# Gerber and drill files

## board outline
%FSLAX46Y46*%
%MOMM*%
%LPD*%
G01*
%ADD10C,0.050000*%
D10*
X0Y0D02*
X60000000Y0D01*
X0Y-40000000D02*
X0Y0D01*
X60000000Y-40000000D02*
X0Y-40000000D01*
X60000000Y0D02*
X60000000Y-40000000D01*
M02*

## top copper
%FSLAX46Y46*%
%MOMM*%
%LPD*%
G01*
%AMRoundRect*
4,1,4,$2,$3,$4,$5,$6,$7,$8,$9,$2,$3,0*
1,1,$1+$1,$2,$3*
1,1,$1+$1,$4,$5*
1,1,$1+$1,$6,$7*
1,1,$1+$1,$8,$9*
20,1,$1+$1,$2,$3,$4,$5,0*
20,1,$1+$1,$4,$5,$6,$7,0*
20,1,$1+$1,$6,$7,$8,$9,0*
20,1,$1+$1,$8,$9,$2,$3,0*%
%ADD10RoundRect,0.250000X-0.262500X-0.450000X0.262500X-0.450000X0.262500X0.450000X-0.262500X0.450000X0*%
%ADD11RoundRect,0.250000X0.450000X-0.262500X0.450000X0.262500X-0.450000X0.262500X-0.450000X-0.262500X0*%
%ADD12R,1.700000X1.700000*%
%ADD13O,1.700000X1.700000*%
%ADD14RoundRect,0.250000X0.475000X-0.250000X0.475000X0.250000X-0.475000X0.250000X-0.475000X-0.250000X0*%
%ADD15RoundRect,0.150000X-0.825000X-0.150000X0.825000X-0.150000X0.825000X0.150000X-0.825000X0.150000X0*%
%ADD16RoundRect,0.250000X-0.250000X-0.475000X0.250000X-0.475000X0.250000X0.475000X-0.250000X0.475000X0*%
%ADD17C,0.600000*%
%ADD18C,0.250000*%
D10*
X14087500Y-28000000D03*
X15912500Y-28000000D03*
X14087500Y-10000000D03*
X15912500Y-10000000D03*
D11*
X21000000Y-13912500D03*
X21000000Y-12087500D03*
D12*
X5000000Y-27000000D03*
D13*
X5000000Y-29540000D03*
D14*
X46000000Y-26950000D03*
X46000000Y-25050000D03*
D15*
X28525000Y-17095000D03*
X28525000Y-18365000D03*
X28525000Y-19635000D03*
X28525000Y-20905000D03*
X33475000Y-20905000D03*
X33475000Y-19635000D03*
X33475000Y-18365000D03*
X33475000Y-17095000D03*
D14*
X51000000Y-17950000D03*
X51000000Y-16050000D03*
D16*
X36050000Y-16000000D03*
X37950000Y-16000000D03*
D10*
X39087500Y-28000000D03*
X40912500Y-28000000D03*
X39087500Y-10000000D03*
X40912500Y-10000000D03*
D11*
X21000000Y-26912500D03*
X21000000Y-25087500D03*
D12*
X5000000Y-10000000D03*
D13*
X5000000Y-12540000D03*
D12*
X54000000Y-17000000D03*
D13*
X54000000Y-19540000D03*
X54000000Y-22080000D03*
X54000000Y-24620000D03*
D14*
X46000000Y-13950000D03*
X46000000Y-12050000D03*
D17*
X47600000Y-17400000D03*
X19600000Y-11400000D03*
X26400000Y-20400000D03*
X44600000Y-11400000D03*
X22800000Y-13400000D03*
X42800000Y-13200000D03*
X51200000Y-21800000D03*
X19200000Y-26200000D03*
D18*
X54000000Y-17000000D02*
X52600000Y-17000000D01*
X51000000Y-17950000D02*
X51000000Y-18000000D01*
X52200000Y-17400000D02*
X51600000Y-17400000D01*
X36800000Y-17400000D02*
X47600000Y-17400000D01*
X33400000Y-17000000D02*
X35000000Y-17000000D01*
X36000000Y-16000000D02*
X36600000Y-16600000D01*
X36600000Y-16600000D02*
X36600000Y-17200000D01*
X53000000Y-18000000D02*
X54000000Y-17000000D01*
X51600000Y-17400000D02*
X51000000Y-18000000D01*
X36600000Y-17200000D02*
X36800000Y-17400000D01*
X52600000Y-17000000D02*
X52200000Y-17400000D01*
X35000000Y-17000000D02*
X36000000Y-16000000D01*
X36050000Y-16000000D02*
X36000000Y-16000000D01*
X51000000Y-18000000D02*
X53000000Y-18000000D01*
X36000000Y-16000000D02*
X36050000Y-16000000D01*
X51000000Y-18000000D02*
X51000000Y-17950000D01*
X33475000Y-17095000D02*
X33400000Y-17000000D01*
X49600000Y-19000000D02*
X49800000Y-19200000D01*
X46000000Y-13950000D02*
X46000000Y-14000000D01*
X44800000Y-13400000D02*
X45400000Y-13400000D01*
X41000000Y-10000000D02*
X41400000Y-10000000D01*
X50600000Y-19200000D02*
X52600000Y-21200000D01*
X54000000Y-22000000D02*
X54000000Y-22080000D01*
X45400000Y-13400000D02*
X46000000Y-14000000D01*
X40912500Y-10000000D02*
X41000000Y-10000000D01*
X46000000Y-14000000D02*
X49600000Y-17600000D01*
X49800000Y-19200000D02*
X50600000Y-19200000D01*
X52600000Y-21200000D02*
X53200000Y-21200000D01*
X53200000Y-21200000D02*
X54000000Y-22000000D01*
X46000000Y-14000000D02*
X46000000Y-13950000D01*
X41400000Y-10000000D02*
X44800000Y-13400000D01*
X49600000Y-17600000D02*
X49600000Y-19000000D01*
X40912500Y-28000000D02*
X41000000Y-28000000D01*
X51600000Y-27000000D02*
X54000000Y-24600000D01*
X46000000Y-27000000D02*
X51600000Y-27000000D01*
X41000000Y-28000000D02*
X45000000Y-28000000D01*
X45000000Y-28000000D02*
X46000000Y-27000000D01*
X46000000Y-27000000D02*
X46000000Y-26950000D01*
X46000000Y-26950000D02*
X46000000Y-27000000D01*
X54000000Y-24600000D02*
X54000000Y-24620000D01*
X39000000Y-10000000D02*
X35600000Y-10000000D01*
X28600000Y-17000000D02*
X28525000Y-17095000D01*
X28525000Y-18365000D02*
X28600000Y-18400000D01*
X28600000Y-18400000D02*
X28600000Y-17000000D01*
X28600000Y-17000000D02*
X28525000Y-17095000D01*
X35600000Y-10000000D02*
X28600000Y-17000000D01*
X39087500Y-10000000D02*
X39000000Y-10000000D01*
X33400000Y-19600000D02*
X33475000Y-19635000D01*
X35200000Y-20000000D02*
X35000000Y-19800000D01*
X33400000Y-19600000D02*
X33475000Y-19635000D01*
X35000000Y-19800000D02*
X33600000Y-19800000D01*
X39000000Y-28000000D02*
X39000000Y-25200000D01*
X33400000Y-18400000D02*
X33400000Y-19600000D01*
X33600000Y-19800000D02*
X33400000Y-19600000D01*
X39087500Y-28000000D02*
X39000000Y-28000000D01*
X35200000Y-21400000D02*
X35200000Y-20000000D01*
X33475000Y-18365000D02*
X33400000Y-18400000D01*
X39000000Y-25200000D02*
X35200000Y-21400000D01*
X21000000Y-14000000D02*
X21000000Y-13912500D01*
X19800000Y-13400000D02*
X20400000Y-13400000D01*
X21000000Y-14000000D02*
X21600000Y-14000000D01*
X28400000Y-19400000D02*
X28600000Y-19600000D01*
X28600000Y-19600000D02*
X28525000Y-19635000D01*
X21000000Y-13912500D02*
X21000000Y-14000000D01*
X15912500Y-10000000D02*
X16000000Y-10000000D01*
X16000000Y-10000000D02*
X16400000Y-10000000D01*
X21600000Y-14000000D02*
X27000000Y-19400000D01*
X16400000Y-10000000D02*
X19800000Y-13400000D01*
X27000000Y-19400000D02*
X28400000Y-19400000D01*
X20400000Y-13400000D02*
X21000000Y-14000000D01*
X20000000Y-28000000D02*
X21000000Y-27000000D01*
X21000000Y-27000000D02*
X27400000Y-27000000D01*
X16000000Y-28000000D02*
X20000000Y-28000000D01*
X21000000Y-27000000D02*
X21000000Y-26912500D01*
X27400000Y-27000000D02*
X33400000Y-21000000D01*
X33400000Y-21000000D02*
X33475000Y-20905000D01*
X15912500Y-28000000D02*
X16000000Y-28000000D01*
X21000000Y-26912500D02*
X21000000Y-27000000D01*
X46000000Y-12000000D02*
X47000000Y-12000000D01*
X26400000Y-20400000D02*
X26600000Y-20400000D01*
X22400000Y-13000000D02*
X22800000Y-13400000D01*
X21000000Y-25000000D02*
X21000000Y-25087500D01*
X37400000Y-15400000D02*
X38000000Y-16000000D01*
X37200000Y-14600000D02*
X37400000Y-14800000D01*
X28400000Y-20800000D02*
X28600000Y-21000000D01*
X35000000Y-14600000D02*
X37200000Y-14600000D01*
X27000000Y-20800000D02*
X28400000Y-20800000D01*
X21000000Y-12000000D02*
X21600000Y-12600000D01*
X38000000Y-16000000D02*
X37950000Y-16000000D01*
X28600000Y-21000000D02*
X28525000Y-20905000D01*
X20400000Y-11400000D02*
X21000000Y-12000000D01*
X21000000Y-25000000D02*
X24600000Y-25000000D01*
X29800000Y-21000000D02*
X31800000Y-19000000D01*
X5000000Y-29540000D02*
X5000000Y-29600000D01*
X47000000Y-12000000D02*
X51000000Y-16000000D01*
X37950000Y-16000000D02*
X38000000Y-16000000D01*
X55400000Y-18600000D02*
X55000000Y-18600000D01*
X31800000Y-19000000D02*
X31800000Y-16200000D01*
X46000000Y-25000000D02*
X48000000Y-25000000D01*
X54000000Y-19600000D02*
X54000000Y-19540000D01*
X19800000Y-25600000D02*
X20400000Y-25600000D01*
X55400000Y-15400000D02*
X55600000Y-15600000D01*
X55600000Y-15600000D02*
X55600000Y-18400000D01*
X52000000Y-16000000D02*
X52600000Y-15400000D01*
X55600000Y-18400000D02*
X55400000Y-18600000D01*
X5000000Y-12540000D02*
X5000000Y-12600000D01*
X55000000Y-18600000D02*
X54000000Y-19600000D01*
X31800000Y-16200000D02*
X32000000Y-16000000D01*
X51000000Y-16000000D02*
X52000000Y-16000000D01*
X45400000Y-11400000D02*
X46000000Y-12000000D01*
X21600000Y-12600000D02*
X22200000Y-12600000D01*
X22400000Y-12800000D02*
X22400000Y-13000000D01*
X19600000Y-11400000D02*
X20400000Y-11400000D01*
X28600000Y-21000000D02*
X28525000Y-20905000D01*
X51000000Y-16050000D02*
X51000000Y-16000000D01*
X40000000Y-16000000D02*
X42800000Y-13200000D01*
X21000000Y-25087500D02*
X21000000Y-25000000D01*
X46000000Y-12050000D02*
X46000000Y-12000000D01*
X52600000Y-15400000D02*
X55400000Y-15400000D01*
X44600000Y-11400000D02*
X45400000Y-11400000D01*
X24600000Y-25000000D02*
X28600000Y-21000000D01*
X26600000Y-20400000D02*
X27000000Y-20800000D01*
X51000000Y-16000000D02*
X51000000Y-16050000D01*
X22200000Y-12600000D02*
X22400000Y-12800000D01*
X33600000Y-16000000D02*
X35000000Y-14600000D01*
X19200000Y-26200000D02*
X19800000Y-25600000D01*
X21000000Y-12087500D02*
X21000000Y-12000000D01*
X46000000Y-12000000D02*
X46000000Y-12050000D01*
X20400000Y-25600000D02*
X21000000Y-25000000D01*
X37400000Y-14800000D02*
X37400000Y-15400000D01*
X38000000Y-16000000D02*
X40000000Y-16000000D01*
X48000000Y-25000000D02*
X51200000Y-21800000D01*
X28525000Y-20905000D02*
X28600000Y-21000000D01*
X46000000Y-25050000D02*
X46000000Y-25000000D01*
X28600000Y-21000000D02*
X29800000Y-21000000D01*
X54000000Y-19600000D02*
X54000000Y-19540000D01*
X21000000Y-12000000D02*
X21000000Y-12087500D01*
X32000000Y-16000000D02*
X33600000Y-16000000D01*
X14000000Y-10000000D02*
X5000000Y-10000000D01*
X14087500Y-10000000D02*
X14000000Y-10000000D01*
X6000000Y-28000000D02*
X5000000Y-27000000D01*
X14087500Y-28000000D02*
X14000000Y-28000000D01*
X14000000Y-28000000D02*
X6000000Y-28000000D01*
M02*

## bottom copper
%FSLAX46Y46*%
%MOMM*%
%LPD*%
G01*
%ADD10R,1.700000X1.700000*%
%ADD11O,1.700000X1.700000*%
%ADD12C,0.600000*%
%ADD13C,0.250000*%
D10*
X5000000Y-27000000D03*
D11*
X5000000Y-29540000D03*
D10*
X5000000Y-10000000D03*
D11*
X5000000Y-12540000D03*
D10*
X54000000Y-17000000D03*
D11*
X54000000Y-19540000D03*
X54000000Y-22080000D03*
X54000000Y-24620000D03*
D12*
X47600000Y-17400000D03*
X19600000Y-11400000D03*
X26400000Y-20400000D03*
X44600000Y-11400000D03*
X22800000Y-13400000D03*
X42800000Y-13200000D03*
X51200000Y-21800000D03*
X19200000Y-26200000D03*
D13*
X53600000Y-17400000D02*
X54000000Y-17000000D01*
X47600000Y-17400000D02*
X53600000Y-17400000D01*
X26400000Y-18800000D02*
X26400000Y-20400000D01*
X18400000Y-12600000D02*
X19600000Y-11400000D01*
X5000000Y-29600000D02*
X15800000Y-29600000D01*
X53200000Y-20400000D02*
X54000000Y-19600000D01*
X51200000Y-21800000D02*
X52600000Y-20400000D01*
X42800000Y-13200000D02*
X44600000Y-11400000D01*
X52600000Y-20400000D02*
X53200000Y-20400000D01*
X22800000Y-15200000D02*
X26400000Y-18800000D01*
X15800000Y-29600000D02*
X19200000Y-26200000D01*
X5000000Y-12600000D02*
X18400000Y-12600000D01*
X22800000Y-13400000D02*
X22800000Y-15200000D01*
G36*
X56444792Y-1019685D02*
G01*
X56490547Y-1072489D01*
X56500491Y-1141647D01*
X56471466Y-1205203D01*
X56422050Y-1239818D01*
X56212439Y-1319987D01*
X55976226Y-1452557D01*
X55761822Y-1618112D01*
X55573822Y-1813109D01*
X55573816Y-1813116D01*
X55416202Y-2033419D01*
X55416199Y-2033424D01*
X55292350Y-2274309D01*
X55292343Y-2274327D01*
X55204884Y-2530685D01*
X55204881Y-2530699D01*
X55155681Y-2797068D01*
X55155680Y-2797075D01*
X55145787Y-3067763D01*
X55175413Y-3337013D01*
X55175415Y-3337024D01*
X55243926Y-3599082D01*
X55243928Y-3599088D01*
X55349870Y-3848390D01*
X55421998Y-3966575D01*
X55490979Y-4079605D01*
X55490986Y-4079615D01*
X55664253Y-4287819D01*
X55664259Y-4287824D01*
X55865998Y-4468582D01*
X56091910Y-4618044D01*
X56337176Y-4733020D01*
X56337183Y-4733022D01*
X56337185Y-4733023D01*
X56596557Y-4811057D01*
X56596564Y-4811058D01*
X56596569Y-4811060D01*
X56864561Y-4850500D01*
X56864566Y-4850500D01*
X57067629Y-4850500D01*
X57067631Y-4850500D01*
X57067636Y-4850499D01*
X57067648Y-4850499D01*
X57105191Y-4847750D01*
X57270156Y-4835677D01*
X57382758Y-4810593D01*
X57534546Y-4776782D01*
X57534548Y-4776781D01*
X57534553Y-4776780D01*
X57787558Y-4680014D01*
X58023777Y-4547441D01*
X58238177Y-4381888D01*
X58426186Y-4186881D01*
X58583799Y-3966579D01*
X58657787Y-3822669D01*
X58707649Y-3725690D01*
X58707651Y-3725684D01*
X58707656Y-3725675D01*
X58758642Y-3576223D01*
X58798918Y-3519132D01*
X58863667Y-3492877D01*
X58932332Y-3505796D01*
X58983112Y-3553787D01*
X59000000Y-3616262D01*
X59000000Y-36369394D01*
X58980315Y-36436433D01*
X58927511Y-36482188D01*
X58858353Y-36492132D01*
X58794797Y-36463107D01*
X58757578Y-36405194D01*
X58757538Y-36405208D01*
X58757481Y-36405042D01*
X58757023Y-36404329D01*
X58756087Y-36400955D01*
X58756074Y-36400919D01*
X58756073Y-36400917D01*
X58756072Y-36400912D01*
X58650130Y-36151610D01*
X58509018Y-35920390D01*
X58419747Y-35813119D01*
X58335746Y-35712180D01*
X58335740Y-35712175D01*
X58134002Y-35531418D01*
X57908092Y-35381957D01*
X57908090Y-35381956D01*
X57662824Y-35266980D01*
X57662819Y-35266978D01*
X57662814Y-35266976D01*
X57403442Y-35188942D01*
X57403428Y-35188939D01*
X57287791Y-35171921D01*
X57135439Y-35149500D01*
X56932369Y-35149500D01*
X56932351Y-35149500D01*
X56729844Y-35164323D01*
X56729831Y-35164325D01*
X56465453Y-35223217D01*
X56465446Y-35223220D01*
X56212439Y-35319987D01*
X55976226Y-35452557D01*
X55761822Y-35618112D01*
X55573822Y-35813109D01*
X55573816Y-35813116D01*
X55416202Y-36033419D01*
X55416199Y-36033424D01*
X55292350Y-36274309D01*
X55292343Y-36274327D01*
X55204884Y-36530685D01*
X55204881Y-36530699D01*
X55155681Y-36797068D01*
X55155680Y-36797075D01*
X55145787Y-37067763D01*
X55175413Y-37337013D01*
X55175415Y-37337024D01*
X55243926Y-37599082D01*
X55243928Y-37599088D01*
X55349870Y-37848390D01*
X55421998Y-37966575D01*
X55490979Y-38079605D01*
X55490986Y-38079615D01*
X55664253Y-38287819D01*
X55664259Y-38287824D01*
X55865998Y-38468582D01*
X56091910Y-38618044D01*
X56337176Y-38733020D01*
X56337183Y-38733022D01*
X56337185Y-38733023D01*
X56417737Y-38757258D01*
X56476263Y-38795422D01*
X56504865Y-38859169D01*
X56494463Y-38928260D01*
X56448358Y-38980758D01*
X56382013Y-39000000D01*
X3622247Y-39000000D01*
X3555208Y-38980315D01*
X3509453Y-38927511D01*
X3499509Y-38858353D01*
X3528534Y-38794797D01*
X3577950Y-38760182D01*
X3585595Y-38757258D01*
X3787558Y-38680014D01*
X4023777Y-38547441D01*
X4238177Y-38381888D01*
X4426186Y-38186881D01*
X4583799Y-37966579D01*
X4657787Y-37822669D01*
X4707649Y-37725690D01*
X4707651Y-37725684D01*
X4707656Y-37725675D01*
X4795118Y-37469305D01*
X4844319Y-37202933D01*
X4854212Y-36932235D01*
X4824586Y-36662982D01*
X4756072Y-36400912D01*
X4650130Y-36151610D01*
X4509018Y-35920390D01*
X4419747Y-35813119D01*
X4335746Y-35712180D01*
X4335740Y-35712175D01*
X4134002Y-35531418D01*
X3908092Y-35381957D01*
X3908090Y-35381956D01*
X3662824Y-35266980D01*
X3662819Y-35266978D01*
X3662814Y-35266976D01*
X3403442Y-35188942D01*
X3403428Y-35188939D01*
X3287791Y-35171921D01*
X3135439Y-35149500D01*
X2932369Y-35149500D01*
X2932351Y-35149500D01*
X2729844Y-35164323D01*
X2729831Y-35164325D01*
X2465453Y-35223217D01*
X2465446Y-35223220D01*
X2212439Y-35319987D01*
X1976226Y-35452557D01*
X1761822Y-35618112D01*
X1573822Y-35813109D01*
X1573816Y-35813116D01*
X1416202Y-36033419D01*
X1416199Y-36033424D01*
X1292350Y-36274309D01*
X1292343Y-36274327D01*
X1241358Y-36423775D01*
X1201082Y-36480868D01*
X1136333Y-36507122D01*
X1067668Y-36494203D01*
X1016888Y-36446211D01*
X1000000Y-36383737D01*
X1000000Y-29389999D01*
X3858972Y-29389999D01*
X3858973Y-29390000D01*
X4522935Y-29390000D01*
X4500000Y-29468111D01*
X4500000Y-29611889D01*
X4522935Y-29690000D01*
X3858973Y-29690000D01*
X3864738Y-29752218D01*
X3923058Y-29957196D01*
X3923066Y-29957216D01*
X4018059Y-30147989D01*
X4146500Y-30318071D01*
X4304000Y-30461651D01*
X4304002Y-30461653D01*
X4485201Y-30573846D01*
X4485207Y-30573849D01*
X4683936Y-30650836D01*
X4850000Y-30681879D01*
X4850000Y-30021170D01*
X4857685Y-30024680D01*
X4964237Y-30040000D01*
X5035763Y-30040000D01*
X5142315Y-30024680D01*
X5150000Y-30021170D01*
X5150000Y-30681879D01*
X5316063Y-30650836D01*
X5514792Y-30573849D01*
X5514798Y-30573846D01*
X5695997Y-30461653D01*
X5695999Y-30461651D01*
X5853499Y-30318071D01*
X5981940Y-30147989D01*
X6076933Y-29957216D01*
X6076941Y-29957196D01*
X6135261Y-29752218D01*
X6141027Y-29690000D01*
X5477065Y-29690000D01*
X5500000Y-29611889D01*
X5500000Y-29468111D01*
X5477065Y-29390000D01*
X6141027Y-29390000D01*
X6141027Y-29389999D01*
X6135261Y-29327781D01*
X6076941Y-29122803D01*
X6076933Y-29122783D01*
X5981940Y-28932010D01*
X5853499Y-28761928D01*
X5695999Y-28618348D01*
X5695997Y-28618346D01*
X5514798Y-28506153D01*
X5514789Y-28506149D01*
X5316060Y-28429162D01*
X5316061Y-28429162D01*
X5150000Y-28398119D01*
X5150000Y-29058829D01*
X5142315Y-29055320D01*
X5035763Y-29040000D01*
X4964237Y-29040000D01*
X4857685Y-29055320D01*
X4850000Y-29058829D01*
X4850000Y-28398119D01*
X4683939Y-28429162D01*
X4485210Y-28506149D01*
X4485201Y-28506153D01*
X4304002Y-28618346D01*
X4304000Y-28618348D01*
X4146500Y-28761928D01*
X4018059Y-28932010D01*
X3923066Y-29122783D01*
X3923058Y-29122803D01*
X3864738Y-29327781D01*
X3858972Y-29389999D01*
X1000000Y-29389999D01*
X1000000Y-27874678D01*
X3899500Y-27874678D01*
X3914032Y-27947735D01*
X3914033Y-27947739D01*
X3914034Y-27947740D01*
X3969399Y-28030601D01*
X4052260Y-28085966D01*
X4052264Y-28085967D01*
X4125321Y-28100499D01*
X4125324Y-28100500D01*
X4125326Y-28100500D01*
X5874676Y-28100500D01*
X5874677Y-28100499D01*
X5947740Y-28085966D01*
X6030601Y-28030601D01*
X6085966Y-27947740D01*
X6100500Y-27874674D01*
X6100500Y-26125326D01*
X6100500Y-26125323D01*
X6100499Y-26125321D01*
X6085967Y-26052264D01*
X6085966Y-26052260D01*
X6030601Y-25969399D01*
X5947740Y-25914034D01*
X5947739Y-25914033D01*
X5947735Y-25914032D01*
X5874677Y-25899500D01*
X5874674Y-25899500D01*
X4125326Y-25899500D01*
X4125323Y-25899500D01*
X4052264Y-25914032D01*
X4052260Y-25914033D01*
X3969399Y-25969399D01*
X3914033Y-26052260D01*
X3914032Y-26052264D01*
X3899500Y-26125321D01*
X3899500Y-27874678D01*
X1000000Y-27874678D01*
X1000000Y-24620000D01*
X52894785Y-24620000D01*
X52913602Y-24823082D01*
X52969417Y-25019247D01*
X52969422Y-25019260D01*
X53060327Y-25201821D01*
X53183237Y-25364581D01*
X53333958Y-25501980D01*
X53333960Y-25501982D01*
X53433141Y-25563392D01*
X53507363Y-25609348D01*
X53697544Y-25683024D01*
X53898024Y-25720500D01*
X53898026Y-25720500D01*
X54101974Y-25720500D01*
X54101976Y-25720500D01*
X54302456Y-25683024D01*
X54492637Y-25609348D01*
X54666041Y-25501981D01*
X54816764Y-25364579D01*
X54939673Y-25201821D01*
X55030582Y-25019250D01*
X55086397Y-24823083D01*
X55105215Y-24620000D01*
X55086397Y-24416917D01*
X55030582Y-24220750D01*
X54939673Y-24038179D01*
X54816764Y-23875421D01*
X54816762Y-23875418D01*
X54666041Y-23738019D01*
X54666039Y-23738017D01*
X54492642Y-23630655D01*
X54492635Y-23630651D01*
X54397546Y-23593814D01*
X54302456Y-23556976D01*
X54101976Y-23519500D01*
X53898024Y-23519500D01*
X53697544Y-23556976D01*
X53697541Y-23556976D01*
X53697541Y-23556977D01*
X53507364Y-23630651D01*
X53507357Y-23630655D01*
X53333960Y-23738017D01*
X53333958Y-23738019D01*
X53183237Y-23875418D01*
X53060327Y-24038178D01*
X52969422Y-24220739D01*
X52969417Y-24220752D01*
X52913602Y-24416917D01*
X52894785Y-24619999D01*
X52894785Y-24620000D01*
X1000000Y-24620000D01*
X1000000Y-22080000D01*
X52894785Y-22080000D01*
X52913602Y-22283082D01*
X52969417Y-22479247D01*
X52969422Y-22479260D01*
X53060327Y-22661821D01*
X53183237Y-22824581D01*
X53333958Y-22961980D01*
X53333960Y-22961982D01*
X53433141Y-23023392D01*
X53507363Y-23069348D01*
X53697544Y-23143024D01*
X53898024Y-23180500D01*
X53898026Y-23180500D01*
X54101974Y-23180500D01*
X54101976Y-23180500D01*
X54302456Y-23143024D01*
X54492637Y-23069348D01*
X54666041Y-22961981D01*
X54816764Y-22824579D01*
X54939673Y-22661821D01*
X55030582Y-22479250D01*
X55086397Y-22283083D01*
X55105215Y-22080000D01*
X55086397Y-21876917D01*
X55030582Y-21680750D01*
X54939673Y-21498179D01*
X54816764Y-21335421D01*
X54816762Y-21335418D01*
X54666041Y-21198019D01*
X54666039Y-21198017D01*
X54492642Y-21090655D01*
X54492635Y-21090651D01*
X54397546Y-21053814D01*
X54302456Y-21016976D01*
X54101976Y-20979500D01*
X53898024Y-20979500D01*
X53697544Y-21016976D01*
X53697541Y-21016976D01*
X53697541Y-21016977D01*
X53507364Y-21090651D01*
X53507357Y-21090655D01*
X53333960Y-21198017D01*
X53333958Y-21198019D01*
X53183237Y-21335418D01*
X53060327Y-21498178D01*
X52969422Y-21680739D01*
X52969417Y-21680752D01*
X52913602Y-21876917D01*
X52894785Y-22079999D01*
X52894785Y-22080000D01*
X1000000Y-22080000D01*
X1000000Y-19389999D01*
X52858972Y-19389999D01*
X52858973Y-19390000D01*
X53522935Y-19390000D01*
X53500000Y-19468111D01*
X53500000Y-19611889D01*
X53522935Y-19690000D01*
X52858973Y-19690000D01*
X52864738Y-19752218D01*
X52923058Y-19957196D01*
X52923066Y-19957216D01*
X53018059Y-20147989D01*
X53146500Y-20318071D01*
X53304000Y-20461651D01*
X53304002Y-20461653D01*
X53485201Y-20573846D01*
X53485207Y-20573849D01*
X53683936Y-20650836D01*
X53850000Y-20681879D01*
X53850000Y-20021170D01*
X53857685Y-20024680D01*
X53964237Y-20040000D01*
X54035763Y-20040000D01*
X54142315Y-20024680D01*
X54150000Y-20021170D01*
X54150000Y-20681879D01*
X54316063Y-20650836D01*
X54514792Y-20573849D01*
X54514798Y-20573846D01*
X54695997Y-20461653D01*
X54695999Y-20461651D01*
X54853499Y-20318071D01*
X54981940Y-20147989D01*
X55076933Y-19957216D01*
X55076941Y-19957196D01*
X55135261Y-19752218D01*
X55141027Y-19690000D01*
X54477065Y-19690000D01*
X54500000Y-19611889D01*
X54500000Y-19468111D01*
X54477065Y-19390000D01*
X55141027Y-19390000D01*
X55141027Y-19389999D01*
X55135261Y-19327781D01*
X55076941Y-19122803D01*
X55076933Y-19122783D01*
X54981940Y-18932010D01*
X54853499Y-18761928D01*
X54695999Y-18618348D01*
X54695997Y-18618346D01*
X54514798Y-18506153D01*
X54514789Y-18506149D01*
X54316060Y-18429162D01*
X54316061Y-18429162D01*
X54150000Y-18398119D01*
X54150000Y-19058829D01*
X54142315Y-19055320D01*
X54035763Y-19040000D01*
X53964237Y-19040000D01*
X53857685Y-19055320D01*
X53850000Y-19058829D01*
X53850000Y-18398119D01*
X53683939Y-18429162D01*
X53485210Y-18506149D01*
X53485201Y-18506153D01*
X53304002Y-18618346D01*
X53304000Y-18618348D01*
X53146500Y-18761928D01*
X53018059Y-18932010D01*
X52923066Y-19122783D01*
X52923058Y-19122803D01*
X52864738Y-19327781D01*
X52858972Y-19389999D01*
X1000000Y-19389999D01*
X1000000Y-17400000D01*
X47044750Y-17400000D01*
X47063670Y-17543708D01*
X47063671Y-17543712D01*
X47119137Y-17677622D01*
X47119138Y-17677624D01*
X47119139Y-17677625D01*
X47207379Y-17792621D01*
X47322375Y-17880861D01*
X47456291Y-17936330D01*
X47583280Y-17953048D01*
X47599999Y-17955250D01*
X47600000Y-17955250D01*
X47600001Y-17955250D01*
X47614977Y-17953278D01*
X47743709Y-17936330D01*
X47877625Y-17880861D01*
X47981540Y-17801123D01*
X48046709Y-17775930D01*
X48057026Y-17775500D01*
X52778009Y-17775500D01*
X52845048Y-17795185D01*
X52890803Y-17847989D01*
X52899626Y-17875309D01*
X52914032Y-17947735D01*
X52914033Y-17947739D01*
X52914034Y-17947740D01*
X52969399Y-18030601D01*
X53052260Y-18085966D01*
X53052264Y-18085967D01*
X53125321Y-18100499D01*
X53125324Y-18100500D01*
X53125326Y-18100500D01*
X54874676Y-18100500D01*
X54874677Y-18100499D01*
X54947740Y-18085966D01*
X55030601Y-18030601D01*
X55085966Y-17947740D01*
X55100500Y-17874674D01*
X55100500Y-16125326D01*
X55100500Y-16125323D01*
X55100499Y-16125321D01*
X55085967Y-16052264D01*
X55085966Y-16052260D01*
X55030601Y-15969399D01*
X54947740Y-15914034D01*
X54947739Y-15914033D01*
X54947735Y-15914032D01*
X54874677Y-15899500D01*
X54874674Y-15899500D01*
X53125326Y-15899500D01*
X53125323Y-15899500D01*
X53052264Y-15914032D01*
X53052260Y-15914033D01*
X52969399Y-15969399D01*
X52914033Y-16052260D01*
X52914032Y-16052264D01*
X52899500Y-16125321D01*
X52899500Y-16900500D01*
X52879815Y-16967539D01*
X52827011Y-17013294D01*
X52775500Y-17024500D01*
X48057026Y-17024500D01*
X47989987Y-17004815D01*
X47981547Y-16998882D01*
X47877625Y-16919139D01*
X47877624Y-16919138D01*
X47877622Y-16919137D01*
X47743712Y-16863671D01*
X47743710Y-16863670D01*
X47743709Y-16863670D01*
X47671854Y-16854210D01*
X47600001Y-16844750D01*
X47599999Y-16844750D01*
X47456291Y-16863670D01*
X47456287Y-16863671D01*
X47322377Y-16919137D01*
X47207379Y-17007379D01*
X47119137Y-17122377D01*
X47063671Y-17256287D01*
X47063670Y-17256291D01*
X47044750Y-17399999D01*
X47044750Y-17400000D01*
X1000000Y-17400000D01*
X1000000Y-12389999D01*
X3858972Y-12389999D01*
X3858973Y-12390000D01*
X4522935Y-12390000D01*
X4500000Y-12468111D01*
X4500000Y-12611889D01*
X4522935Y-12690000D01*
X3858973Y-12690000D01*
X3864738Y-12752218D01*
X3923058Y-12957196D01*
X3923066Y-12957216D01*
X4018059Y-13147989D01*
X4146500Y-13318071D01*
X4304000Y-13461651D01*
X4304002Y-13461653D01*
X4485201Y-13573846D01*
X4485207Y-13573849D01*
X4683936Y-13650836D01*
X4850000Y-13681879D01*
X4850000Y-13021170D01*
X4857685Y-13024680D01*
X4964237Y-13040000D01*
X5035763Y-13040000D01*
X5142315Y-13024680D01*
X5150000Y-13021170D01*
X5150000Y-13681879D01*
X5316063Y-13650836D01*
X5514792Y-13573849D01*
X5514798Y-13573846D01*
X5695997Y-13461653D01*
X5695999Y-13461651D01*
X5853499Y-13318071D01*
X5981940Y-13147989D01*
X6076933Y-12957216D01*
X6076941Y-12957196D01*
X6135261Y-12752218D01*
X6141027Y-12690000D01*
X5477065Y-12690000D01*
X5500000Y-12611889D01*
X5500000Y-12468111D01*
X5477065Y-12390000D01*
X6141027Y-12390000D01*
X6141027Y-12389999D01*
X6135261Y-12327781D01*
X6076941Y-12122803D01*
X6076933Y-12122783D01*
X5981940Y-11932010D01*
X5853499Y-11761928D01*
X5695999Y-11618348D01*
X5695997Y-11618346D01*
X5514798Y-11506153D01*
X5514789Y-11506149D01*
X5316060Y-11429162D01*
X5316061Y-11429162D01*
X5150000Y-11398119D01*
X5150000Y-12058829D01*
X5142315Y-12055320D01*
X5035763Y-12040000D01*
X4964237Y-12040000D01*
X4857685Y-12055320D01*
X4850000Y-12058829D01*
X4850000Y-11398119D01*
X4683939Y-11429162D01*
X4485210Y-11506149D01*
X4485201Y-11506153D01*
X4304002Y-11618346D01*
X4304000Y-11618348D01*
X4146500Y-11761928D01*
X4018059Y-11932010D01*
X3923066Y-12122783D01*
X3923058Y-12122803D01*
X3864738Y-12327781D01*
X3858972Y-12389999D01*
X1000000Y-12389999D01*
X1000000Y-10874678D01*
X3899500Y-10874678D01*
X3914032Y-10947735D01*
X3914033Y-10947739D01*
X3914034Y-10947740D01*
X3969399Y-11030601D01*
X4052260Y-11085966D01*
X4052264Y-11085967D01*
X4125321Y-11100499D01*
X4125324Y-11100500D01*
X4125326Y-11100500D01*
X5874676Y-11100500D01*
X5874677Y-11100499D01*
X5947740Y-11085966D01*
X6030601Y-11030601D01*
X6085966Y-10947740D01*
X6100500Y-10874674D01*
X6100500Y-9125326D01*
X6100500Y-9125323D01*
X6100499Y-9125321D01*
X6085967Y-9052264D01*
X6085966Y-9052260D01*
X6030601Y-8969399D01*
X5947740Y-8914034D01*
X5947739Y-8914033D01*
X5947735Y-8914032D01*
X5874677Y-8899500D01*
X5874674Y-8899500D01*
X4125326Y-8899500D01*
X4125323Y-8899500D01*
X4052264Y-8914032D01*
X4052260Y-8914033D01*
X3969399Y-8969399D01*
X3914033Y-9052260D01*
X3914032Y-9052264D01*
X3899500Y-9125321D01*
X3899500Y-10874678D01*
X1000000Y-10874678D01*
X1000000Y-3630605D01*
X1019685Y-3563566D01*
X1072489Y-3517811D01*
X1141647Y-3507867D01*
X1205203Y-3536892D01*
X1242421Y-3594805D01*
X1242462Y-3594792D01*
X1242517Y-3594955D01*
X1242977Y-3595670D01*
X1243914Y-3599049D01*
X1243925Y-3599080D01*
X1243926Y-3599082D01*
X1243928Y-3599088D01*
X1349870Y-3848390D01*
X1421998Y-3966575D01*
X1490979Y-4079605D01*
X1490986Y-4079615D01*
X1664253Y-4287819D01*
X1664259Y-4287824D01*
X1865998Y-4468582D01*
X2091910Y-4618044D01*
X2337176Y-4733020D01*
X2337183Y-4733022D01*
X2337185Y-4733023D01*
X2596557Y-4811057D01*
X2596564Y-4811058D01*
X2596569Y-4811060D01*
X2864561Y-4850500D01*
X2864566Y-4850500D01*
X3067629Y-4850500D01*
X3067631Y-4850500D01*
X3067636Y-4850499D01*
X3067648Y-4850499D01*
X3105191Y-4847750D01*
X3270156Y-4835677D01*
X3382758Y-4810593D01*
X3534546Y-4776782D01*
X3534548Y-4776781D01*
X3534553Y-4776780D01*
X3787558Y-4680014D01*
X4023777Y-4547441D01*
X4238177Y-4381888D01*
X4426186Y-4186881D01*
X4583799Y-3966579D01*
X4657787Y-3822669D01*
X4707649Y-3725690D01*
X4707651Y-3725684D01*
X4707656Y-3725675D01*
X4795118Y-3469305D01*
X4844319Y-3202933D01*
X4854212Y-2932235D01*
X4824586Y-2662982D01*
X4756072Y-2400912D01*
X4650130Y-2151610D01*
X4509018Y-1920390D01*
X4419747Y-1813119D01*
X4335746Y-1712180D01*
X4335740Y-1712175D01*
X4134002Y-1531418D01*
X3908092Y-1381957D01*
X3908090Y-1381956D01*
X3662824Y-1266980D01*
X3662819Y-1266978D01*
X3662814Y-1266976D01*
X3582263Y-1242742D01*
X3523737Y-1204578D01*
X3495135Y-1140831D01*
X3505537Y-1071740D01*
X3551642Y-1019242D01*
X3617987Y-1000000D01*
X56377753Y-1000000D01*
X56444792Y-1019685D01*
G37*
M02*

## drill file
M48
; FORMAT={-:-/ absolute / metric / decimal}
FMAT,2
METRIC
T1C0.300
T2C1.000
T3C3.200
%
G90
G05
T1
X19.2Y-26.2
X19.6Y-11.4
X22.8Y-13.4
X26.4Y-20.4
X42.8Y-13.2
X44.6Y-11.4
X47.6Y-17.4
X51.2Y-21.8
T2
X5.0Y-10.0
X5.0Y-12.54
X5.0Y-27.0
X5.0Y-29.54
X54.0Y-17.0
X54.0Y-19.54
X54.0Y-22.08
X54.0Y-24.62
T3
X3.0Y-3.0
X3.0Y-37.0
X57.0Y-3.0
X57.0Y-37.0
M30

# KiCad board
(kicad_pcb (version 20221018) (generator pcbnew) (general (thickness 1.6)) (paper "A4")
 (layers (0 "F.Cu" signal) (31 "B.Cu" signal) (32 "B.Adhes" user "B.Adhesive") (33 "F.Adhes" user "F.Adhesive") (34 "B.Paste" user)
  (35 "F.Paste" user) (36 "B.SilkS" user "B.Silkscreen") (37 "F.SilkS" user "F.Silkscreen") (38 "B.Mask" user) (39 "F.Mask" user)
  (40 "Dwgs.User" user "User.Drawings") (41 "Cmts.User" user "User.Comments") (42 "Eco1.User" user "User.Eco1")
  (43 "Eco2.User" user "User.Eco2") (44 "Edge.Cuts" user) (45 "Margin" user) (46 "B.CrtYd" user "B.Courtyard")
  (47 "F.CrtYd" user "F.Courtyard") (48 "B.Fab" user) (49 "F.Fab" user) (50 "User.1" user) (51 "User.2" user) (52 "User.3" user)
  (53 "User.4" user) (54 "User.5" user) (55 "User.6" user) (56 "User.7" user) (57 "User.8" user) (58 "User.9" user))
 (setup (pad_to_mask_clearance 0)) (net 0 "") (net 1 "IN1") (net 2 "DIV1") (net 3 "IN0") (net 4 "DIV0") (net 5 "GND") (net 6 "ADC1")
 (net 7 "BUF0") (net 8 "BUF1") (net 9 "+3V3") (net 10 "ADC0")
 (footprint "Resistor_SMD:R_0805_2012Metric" (layer "F.Cu") (at 15 28)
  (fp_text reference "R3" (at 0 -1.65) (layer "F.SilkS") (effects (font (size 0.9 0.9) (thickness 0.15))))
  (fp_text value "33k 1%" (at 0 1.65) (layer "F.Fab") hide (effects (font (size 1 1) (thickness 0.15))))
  (pad "1" smd roundrect (at -0.9125 0) (size 1.025 1.4) (layers "F.Cu" "F.Paste" "F.Mask") (roundrect_rratio 0.243902) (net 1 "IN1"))
  (pad "2" smd roundrect (at 0.9125 0) (size 1.025 1.4) (layers "F.Cu" "F.Paste" "F.Mask") (roundrect_rratio 0.243902) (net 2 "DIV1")))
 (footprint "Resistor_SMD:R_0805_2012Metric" (layer "F.Cu") (at 15 10)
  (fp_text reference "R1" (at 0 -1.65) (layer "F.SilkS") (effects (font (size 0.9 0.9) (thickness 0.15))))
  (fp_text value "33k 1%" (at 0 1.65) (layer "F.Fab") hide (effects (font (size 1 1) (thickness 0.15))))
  (pad "1" smd roundrect (at -0.9125 0) (size 1.025 1.4) (layers "F.Cu" "F.Paste" "F.Mask") (roundrect_rratio 0.243902) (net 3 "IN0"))
  (pad "2" smd roundrect (at 0.9125 0) (size 1.025 1.4) (layers "F.Cu" "F.Paste" "F.Mask") (roundrect_rratio 0.243902) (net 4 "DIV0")))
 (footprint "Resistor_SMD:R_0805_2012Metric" (layer "F.Cu") (at 21 13 90)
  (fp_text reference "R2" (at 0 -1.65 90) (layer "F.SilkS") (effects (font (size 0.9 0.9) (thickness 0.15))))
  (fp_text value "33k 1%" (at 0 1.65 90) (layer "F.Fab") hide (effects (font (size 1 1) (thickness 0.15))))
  (pad "1" smd roundrect (at -0.9125 0 90) (size 1.025 1.4) (layers "F.Cu" "F.Paste" "F.Mask") (roundrect_rratio 0.243902) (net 4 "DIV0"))
  (pad "2" smd roundrect (at 0.9125 0 90) (size 1.025 1.4) (layers "F.Cu" "F.Paste" "F.Mask") (roundrect_rratio 0.243902) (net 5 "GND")))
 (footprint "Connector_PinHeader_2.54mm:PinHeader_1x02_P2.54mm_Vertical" (layer "F.Cu") (at 5 27)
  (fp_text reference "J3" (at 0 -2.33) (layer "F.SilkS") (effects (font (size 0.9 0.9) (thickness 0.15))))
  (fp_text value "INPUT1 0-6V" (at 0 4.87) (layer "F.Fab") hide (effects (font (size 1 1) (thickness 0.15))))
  (pad "1" thru_hole rect (at 0 0) (size 1.7 1.7) (drill 1) (layers "*.Cu" "*.Mask") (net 1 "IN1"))
  (pad "2" thru_hole oval (at 0 2.54) (size 1.7 1.7) (drill 1) (layers "*.Cu" "*.Mask") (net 5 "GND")))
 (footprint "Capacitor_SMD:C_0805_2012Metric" (layer "F.Cu") (at 46 26 90)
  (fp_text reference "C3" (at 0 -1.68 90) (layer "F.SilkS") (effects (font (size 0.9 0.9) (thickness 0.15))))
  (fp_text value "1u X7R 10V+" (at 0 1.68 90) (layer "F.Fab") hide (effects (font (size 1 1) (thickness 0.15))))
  (pad "1" smd roundrect (at -0.95 0 90) (size 1 1.45) (layers "F.Cu" "F.Paste" "F.Mask") (roundrect_rratio 0.25) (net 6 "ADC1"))
  (pad "2" smd roundrect (at 0.95 0 90) (size 1 1.45) (layers "F.Cu" "F.Paste" "F.Mask") (roundrect_rratio 0.25) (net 5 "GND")))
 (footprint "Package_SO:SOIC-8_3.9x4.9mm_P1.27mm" (layer "F.Cu") (at 31 19)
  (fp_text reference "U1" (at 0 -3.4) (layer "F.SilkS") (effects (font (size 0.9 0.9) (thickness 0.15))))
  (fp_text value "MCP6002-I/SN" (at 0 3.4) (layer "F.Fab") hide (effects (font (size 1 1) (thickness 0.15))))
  (pad "1" smd roundrect (at -2.475 -1.905) (size 1.95 0.6) (layers "F.Cu" "F.Paste" "F.Mask") (roundrect_rratio 0.25) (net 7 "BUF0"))
  (pad "2" smd roundrect (at -2.475 -0.635) (size 1.95 0.6) (layers "F.Cu" "F.Paste" "F.Mask") (roundrect_rratio 0.25) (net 7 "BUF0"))
  (pad "3" smd roundrect (at -2.475 0.635) (size 1.95 0.6) (layers "F.Cu" "F.Paste" "F.Mask") (roundrect_rratio 0.25) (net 4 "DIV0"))
  (pad "4" smd roundrect (at -2.475 1.905) (size 1.95 0.6) (layers "F.Cu" "F.Paste" "F.Mask") (roundrect_rratio 0.25) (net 5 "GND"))
  (pad "5" smd roundrect (at 2.475 1.905) (size 1.95 0.6) (layers "F.Cu" "F.Paste" "F.Mask") (roundrect_rratio 0.25) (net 2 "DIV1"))
  (pad "6" smd roundrect (at 2.475 0.635) (size 1.95 0.6) (layers "F.Cu" "F.Paste" "F.Mask") (roundrect_rratio 0.25) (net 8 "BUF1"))
  (pad "7" smd roundrect (at 2.475 -0.635) (size 1.95 0.6) (layers "F.Cu" "F.Paste" "F.Mask") (roundrect_rratio 0.25) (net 8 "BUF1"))
  (pad "8" smd roundrect (at 2.475 -1.905) (size 1.95 0.6) (layers "F.Cu" "F.Paste" "F.Mask") (roundrect_rratio 0.25) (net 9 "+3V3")))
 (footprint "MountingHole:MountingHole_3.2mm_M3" (layer "F.Cu") (at 57 3)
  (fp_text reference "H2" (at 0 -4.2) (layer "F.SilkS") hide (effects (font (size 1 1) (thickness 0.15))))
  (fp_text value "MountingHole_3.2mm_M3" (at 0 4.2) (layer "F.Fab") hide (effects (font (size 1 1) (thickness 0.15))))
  (pad "" np_thru_hole circle (at 0 0) (size 3.2 3.2) (drill 3.2) (layers "*.Cu" "*.Mask")))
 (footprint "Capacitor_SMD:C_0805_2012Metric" (layer "F.Cu") (at 51 17 90)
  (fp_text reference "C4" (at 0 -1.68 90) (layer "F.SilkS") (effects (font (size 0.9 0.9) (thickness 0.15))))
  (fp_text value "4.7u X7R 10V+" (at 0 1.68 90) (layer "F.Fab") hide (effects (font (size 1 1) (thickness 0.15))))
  (pad "1" smd roundrect (at -0.95 0 90) (size 1 1.45) (layers "F.Cu" "F.Paste" "F.Mask") (roundrect_rratio 0.25) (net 9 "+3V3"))
  (pad "2" smd roundrect (at 0.95 0 90) (size 1 1.45) (layers "F.Cu" "F.Paste" "F.Mask") (roundrect_rratio 0.25) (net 5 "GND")))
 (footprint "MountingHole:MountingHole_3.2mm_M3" (layer "F.Cu") (at 3 3)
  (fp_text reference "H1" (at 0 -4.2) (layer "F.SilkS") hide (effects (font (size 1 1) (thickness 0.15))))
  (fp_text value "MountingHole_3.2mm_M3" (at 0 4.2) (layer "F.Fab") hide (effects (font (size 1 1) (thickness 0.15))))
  (pad "" np_thru_hole circle (at 0 0) (size 3.2 3.2) (drill 3.2) (layers "*.Cu" "*.Mask")))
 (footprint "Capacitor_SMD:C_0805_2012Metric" (layer "F.Cu") (at 37 16)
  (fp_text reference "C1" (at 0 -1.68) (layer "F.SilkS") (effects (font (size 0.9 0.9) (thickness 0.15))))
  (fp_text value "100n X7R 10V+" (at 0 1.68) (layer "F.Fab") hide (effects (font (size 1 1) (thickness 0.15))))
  (pad "1" smd roundrect (at -0.95 0) (size 1 1.45) (layers "F.Cu" "F.Paste" "F.Mask") (roundrect_rratio 0.25) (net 9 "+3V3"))
  (pad "2" smd roundrect (at 0.95 0) (size 1 1.45) (layers "F.Cu" "F.Paste" "F.Mask") (roundrect_rratio 0.25) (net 5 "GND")))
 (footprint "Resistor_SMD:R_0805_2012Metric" (layer "F.Cu") (at 40 28)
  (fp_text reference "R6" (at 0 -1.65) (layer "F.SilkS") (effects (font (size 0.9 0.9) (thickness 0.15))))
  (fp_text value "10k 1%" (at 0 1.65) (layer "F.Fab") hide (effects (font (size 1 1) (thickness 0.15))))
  (pad "1" smd roundrect (at -0.9125 0) (size 1.025 1.4) (layers "F.Cu" "F.Paste" "F.Mask") (roundrect_rratio 0.243902) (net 8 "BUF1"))
  (pad "2" smd roundrect (at 0.9125 0) (size 1.025 1.4) (layers "F.Cu" "F.Paste" "F.Mask") (roundrect_rratio 0.243902) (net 6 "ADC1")))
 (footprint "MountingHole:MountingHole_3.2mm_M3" (layer "F.Cu") (at 3 37)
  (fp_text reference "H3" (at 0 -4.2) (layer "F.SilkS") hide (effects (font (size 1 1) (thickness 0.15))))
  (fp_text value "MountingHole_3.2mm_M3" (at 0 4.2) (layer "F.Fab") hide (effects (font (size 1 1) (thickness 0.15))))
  (pad "" np_thru_hole circle (at 0 0) (size 3.2 3.2) (drill 3.2) (layers "*.Cu" "*.Mask")))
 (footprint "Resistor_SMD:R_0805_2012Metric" (layer "F.Cu") (at 40 10)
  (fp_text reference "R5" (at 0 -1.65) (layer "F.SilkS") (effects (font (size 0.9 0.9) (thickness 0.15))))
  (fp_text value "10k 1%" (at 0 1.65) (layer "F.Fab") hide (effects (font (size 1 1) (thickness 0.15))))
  (pad "1" smd roundrect (at -0.9125 0) (size 1.025 1.4) (layers "F.Cu" "F.Paste" "F.Mask") (roundrect_rratio 0.243902) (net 7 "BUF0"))
  (pad "2" smd roundrect (at 0.9125 0) (size 1.025 1.4) (layers "F.Cu" "F.Paste" "F.Mask") (roundrect_rratio 0.243902) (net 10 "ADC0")))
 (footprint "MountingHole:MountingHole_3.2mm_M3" (layer "F.Cu") (at 57 37)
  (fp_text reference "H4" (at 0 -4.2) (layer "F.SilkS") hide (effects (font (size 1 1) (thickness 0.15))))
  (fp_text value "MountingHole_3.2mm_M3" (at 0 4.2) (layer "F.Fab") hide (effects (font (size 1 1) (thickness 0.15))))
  (pad "" np_thru_hole circle (at 0 0) (size 3.2 3.2) (drill 3.2) (layers "*.Cu" "*.Mask")))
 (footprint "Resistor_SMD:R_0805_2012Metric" (layer "F.Cu") (at 21 26 90)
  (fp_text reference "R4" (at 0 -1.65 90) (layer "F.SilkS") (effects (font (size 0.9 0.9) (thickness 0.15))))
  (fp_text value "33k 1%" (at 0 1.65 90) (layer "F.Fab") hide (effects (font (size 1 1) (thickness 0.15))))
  (pad "1" smd roundrect (at -0.9125 0 90) (size 1.025 1.4) (layers "F.Cu" "F.Paste" "F.Mask") (roundrect_rratio 0.243902) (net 2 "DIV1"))
  (pad "2" smd roundrect (at 0.9125 0 90) (size 1.025 1.4) (layers "F.Cu" "F.Paste" "F.Mask") (roundrect_rratio 0.243902) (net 5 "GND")))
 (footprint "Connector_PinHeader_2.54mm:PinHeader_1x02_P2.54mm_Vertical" (layer "F.Cu") (at 5 10)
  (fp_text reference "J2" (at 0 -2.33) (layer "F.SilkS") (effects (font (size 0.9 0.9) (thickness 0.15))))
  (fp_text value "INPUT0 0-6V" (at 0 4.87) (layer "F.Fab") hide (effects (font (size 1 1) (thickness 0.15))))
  (pad "1" thru_hole rect (at 0 0) (size 1.7 1.7) (drill 1) (layers "*.Cu" "*.Mask") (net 3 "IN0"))
  (pad "2" thru_hole oval (at 0 2.54) (size 1.7 1.7) (drill 1) (layers "*.Cu" "*.Mask") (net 5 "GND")))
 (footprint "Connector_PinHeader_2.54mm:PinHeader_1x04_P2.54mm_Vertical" (layer "F.Cu") (at 54 17)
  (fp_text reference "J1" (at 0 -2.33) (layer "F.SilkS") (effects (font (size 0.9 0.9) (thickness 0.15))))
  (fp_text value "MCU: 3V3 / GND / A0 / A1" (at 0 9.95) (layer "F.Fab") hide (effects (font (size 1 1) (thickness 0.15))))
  (pad "1" thru_hole rect (at 0 0) (size 1.7 1.7) (drill 1) (layers "*.Cu" "*.Mask") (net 9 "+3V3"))
  (pad "2" thru_hole oval (at 0 2.54) (size 1.7 1.7) (drill 1) (layers "*.Cu" "*.Mask") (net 5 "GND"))
  (pad "3" thru_hole oval (at 0 5.08) (size 1.7 1.7) (drill 1) (layers "*.Cu" "*.Mask") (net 10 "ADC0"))
  (pad "4" thru_hole oval (at 0 7.62) (size 1.7 1.7) (drill 1) (layers "*.Cu" "*.Mask") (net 6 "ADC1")))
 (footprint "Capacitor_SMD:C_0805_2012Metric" (layer "F.Cu") (at 46 13 90)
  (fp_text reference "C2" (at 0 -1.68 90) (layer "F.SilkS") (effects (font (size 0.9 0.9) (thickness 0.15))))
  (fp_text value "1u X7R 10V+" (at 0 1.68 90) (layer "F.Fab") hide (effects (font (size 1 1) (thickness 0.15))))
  (pad "1" smd roundrect (at -0.95 0 90) (size 1 1.45) (layers "F.Cu" "F.Paste" "F.Mask") (roundrect_rratio 0.25) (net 10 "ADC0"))
  (pad "2" smd roundrect (at 0.95 0 90) (size 1 1.45) (layers "F.Cu" "F.Paste" "F.Mask") (roundrect_rratio 0.25) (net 5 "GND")))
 (gr_line (start 0 0) (end 60 0) (stroke (width 0.05) (type default)) (layer "Edge.Cuts"))
 (gr_line (start 0 40) (end 0 0) (stroke (width 0.05) (type default)) (layer "Edge.Cuts"))
 (gr_line (start 60 40) (end 0 40) (stroke (width 0.05) (type default)) (layer "Edge.Cuts"))
 (gr_line (start 60 0) (end 60 40) (stroke (width 0.05) (type default)) (layer "Edge.Cuts"))
 (segment (start 54 17) (end 52.6 17) (width 0.25) (layer "F.Cu") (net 9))
 (segment (start 51 17.95) (end 51 18) (width 0.25) (layer "F.Cu") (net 9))
 (segment (start 52.2 17.4) (end 51.6 17.4) (width 0.25) (layer "F.Cu") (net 9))
 (segment (start 36.8 17.4) (end 47.6 17.4) (width 0.25) (layer "F.Cu") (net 9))
 (segment (start 33.4 17) (end 35 17) (width 0.25) (layer "F.Cu") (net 9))
 (segment (start 36 16) (end 36.6 16.6) (width 0.25) (layer "F.Cu") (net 9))
 (segment (start 36.6 16.6) (end 36.6 17.2) (width 0.25) (layer "F.Cu") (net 9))
 (segment (start 53 18) (end 54 17) (width 0.25) (layer "F.Cu") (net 9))
 (segment (start 51.6 17.4) (end 51 18) (width 0.25) (layer "F.Cu") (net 9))
 (segment (start 36.6 17.2) (end 36.8 17.4) (width 0.25) (layer "F.Cu") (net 9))
 (segment (start 52.6 17) (end 52.2 17.4) (width 0.25) (layer "F.Cu") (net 9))
 (segment (start 35 17) (end 36 16) (width 0.25) (layer "F.Cu") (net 9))
 (segment (start 36.05 16) (end 36 16) (width 0.25) (layer "F.Cu") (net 9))
 (segment (start 51 18) (end 53 18) (width 0.25) (layer "F.Cu") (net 9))
 (segment (start 36 16) (end 36.05 16) (width 0.25) (layer "F.Cu") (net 9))
 (segment (start 51 18) (end 51 17.95) (width 0.25) (layer "F.Cu") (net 9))
 (segment (start 33.475 17.095) (end 33.4 17) (width 0.25) (layer "F.Cu") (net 9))
 (via (at 47.6 17.4) (size 0.6) (drill 0.3) (layers "F.Cu" "B.Cu") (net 9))
 (segment (start 53.6 17.4) (end 54 17) (width 0.25) (layer "B.Cu") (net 9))
 (segment (start 47.6 17.4) (end 53.6 17.4) (width 0.25) (layer "B.Cu") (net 9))
 (segment (start 49.6 19) (end 49.8 19.2) (width 0.25) (layer "F.Cu") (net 10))
 (segment (start 46 13.95) (end 46 14) (width 0.25) (layer "F.Cu") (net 10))
 (segment (start 44.8 13.4) (end 45.4 13.4) (width 0.25) (layer "F.Cu") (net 10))
 (segment (start 41 10) (end 41.4 10) (width 0.25) (layer "F.Cu") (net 10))
 (segment (start 50.6 19.2) (end 52.6 21.2) (width 0.25) (layer "F.Cu") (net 10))
 (segment (start 54 22) (end 54 22.08) (width 0.25) (layer "F.Cu") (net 10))
 (segment (start 45.4 13.4) (end 46 14) (width 0.25) (layer "F.Cu") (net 10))
 (segment (start 40.9125 10) (end 41 10) (width 0.25) (layer "F.Cu") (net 10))
 (segment (start 46 14) (end 49.6 17.6) (width 0.25) (layer "F.Cu") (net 10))
 (segment (start 49.8 19.2) (end 50.6 19.2) (width 0.25) (layer "F.Cu") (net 10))
 (segment (start 52.6 21.2) (end 53.2 21.2) (width 0.25) (layer "F.Cu") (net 10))
 (segment (start 53.2 21.2) (end 54 22) (width 0.25) (layer "F.Cu") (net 10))
 (segment (start 46 14) (end 46 13.95) (width 0.25) (layer "F.Cu") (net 10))
 (segment (start 41.4 10) (end 44.8 13.4) (width 0.25) (layer "F.Cu") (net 10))
 (segment (start 49.6 17.6) (end 49.6 19) (width 0.25) (layer "F.Cu") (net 10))
 (segment (start 40.9125 28) (end 41 28) (width 0.25) (layer "F.Cu") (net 6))
 (segment (start 51.6 27) (end 54 24.6) (width 0.25) (layer "F.Cu") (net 6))
 (segment (start 46 27) (end 51.6 27) (width 0.25) (layer "F.Cu") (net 6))
 (segment (start 41 28) (end 45 28) (width 0.25) (layer "F.Cu") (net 6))
 (segment (start 45 28) (end 46 27) (width 0.25) (layer "F.Cu") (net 6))
 (segment (start 46 27) (end 46 26.95) (width 0.25) (layer "F.Cu") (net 6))
 (segment (start 46 26.95) (end 46 27) (width 0.25) (layer "F.Cu") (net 6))
 (segment (start 54 24.6) (end 54 24.62) (width 0.25) (layer "F.Cu") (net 6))
 (segment (start 39 10) (end 35.6 10) (width 0.25) (layer "F.Cu") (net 7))
 (segment (start 28.6 17) (end 28.525 17.095) (width 0.25) (layer "F.Cu") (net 7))
 (segment (start 28.525 18.365) (end 28.6 18.4) (width 0.25) (layer "F.Cu") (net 7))
 (segment (start 28.6 18.4) (end 28.6 17) (width 0.25) (layer "F.Cu") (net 7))
 (segment (start 28.6 17) (end 28.525 17.095) (width 0.25) (layer "F.Cu") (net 7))
 (segment (start 35.6 10) (end 28.6 17) (width 0.25) (layer "F.Cu") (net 7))
 (segment (start 39.0875 10) (end 39 10) (width 0.25) (layer "F.Cu") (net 7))
 (segment (start 33.4 19.6) (end 33.475 19.635) (width 0.25) (layer "F.Cu") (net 8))
 (segment (start 35.2 20) (end 35 19.8) (width 0.25) (layer "F.Cu") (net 8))
 (segment (start 33.4 19.6) (end 33.475 19.635) (width 0.25) (layer "F.Cu") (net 8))
 (segment (start 35 19.8) (end 33.6 19.8) (width 0.25) (layer "F.Cu") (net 8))
 (segment (start 39 28) (end 39 25.2) (width 0.25) (layer "F.Cu") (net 8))
 (segment (start 33.4 18.4) (end 33.4 19.6) (width 0.25) (layer "F.Cu") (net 8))
 (segment (start 33.6 19.8) (end 33.4 19.6) (width 0.25) (layer "F.Cu") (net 8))
 (segment (start 39.0875 28) (end 39 28) (width 0.25) (layer "F.Cu") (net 8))
 (segment (start 35.2 21.4) (end 35.2 20) (width 0.25) (layer "F.Cu") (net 8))
 (segment (start 33.475 18.365) (end 33.4 18.4) (width 0.25) (layer "F.Cu") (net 8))
 (segment (start 39 25.2) (end 35.2 21.4) (width 0.25) (layer "F.Cu") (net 8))
 (segment (start 21 14) (end 21 13.9125) (width 0.25) (layer "F.Cu") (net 4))
 (segment (start 19.8 13.4) (end 20.4 13.4) (width 0.25) (layer "F.Cu") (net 4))
 (segment (start 21 14) (end 21.6 14) (width 0.25) (layer "F.Cu") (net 4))
 (segment (start 28.4 19.4) (end 28.6 19.6) (width 0.25) (layer "F.Cu") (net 4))
 (segment (start 28.6 19.6) (end 28.525 19.635) (width 0.25) (layer "F.Cu") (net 4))
 (segment (start 21 13.9125) (end 21 14) (width 0.25) (layer "F.Cu") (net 4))
 (segment (start 15.9125 10) (end 16 10) (width 0.25) (layer "F.Cu") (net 4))
 (segment (start 16 10) (end 16.4 10) (width 0.25) (layer "F.Cu") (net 4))
 (segment (start 21.6 14) (end 27 19.4) (width 0.25) (layer "F.Cu") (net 4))
 (segment (start 16.4 10) (end 19.8 13.4) (width 0.25) (layer "F.Cu") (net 4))
 (segment (start 27 19.4) (end 28.4 19.4) (width 0.25) (layer "F.Cu") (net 4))
 (segment (start 20.4 13.4) (end 21 14) (width 0.25) (layer "F.Cu") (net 4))
 (segment (start 20 28) (end 21 27) (width 0.25) (layer "F.Cu") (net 2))
 (segment (start 21 27) (end 27.4 27) (width 0.25) (layer "F.Cu") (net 2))
 (segment (start 16 28) (end 20 28) (width 0.25) (layer "F.Cu") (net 2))
 (segment (start 21 27) (end 21 26.9125) (width 0.25) (layer "F.Cu") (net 2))
 (segment (start 27.4 27) (end 33.4 21) (width 0.25) (layer "F.Cu") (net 2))
 (segment (start 33.4 21) (end 33.475 20.905) (width 0.25) (layer "F.Cu") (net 2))
 (segment (start 15.9125 28) (end 16 28) (width 0.25) (layer "F.Cu") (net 2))
 (segment (start 21 26.9125) (end 21 27) (width 0.25) (layer "F.Cu") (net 2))
 (segment (start 46 12) (end 47 12) (width 0.25) (layer "F.Cu") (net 5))
 (segment (start 26.4 20.4) (end 26.6 20.4) (width 0.25) (layer "F.Cu") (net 5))
 (segment (start 22.4 13) (end 22.8 13.4) (width 0.25) (layer "F.Cu") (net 5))
 (segment (start 21 25) (end 21 25.0875) (width 0.25) (layer "F.Cu") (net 5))
 (segment (start 37.4 15.4) (end 38 16) (width 0.25) (layer "F.Cu") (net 5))
 (segment (start 37.2 14.6) (end 37.4 14.8) (width 0.25) (layer "F.Cu") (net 5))
 (segment (start 28.4 20.8) (end 28.6 21) (width 0.25) (layer "F.Cu") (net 5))
 (segment (start 35 14.6) (end 37.2 14.6) (width 0.25) (layer "F.Cu") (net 5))
 (segment (start 27 20.8) (end 28.4 20.8) (width 0.25) (layer "F.Cu") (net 5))
 (segment (start 21 12) (end 21.6 12.6) (width 0.25) (layer "F.Cu") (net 5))
 (segment (start 38 16) (end 37.95 16) (width 0.25) (layer "F.Cu") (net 5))
 (segment (start 28.6 21) (end 28.525 20.905) (width 0.25) (layer "F.Cu") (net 5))
 (segment (start 20.4 11.4) (end 21 12) (width 0.25) (layer "F.Cu") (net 5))
 (segment (start 21 25) (end 24.6 25) (width 0.25) (layer "F.Cu") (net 5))
 (segment (start 29.8 21) (end 31.8 19) (width 0.25) (layer "F.Cu") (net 5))
 (segment (start 5 29.54) (end 5 29.6) (width 0.25) (layer "F.Cu") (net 5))
 (segment (start 47 12) (end 51 16) (width 0.25) (layer "F.Cu") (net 5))
 (segment (start 37.95 16) (end 38 16) (width 0.25) (layer "F.Cu") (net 5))
 (segment (start 55.4 18.6) (end 55 18.6) (width 0.25) (layer "F.Cu") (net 5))
 (segment (start 31.8 19) (end 31.8 16.2) (width 0.25) (layer "F.Cu") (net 5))
 (segment (start 46 25) (end 48 25) (width 0.25) (layer "F.Cu") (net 5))
 (segment (start 54 19.6) (end 54 19.54) (width 0.25) (layer "F.Cu") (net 5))
 (segment (start 19.8 25.6) (end 20.4 25.6) (width 0.25) (layer "F.Cu") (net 5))
 (segment (start 55.4 15.4) (end 55.6 15.6) (width 0.25) (layer "F.Cu") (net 5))
 (segment (start 55.6 15.6) (end 55.6 18.4) (width 0.25) (layer "F.Cu") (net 5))
 (segment (start 52 16) (end 52.6 15.4) (width 0.25) (layer "F.Cu") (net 5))
 (segment (start 55.6 18.4) (end 55.4 18.6) (width 0.25) (layer "F.Cu") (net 5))
 (segment (start 5 12.54) (end 5 12.6) (width 0.25) (layer "F.Cu") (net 5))
 (segment (start 55 18.6) (end 54 19.6) (width 0.25) (layer "F.Cu") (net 5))
 (segment (start 31.8 16.2) (end 32 16) (width 0.25) (layer "F.Cu") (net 5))
 (segment (start 51 16) (end 52 16) (width 0.25) (layer "F.Cu") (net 5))
 (segment (start 45.4 11.4) (end 46 12) (width 0.25) (layer "F.Cu") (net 5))
 (segment (start 21.6 12.6) (end 22.2 12.6) (width 0.25) (layer "F.Cu") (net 5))
 (segment (start 22.4 12.8) (end 22.4 13) (width 0.25) (layer "F.Cu") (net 5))
 (segment (start 19.6 11.4) (end 20.4 11.4) (width 0.25) (layer "F.Cu") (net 5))
 (segment (start 28.6 21) (end 28.525 20.905) (width 0.25) (layer "F.Cu") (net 5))
 (segment (start 51 16.05) (end 51 16) (width 0.25) (layer "F.Cu") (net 5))
 (segment (start 40 16) (end 42.8 13.2) (width 0.25) (layer "F.Cu") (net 5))
 (segment (start 21 25.0875) (end 21 25) (width 0.25) (layer "F.Cu") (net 5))
 (segment (start 46 12.05) (end 46 12) (width 0.25) (layer "F.Cu") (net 5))
 (segment (start 52.6 15.4) (end 55.4 15.4) (width 0.25) (layer "F.Cu") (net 5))
 (segment (start 44.6 11.4) (end 45.4 11.4) (width 0.25) (layer "F.Cu") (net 5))
 (segment (start 24.6 25) (end 28.6 21) (width 0.25) (layer "F.Cu") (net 5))
 (segment (start 26.6 20.4) (end 27 20.8) (width 0.25) (layer "F.Cu") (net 5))
 (segment (start 51 16) (end 51 16.05) (width 0.25) (layer "F.Cu") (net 5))
 (segment (start 22.2 12.6) (end 22.4 12.8) (width 0.25) (layer "F.Cu") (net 5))
 (segment (start 33.6 16) (end 35 14.6) (width 0.25) (layer "F.Cu") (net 5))
 (segment (start 19.2 26.2) (end 19.8 25.6) (width 0.25) (layer "F.Cu") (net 5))
 (segment (start 21 12.0875) (end 21 12) (width 0.25) (layer "F.Cu") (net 5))
 (segment (start 46 12) (end 46 12.05) (width 0.25) (layer "F.Cu") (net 5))
 (segment (start 20.4 25.6) (end 21 25) (width 0.25) (layer "F.Cu") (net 5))
 (segment (start 37.4 14.8) (end 37.4 15.4) (width 0.25) (layer "F.Cu") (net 5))
 (segment (start 38 16) (end 40 16) (width 0.25) (layer "F.Cu") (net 5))
 (segment (start 48 25) (end 51.2 21.8) (width 0.25) (layer "F.Cu") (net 5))
 (segment (start 28.525 20.905) (end 28.6 21) (width 0.25) (layer "F.Cu") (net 5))
 (segment (start 46 25.05) (end 46 25) (width 0.25) (layer "F.Cu") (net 5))
 (segment (start 28.6 21) (end 29.8 21) (width 0.25) (layer "F.Cu") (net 5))
 (segment (start 54 19.6) (end 54 19.54) (width 0.25) (layer "F.Cu") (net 5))
 (segment (start 21 12) (end 21 12.0875) (width 0.25) (layer "F.Cu") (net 5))
 (segment (start 32 16) (end 33.6 16) (width 0.25) (layer "F.Cu") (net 5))
 (via (at 19.6 11.4) (size 0.6) (drill 0.3) (layers "F.Cu" "B.Cu") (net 5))
 (via (at 26.4 20.4) (size 0.6) (drill 0.3) (layers "F.Cu" "B.Cu") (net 5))
 (via (at 44.6 11.4) (size 0.6) (drill 0.3) (layers "F.Cu" "B.Cu") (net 5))
 (via (at 22.8 13.4) (size 0.6) (drill 0.3) (layers "F.Cu" "B.Cu") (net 5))
 (via (at 42.8 13.2) (size 0.6) (drill 0.3) (layers "F.Cu" "B.Cu") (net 5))
 (via (at 51.2 21.8) (size 0.6) (drill 0.3) (layers "F.Cu" "B.Cu") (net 5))
 (via (at 19.2 26.2) (size 0.6) (drill 0.3) (layers "F.Cu" "B.Cu") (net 5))
 (segment (start 26.4 18.8) (end 26.4 20.4) (width 0.25) (layer "B.Cu") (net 5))
 (segment (start 18.4 12.6) (end 19.6 11.4) (width 0.25) (layer "B.Cu") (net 5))
 (segment (start 5 29.6) (end 15.8 29.6) (width 0.25) (layer "B.Cu") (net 5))
 (segment (start 53.2 20.4) (end 54 19.6) (width 0.25) (layer "B.Cu") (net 5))
 (segment (start 51.2 21.8) (end 52.6 20.4) (width 0.25) (layer "B.Cu") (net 5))
 (segment (start 42.8 13.2) (end 44.6 11.4) (width 0.25) (layer "B.Cu") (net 5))
 (segment (start 52.6 20.4) (end 53.2 20.4) (width 0.25) (layer "B.Cu") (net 5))
 (segment (start 22.8 15.2) (end 26.4 18.8) (width 0.25) (layer "B.Cu") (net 5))
 (segment (start 15.8 29.6) (end 19.2 26.2) (width 0.25) (layer "B.Cu") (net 5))
 (segment (start 5 12.6) (end 18.4 12.6) (width 0.25) (layer "B.Cu") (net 5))
 (segment (start 22.8 13.4) (end 22.8 15.2) (width 0.25) (layer "B.Cu") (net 5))
 (segment (start 14 10) (end 5 10) (width 0.25) (layer "F.Cu") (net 3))
 (segment (start 14.0875 10) (end 14 10) (width 0.25) (layer "F.Cu") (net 3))
 (segment (start 6 28) (end 5 27) (width 0.25) (layer "F.Cu") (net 1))
 (segment (start 14.0875 28) (end 14 28) (width 0.25) (layer "F.Cu") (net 1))
 (segment (start 14 28) (end 6 28) (width 0.25) (layer "F.Cu") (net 1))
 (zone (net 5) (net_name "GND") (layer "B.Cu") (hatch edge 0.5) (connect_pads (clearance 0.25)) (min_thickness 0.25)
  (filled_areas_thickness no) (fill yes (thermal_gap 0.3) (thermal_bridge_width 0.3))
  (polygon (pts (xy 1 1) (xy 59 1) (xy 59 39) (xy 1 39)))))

